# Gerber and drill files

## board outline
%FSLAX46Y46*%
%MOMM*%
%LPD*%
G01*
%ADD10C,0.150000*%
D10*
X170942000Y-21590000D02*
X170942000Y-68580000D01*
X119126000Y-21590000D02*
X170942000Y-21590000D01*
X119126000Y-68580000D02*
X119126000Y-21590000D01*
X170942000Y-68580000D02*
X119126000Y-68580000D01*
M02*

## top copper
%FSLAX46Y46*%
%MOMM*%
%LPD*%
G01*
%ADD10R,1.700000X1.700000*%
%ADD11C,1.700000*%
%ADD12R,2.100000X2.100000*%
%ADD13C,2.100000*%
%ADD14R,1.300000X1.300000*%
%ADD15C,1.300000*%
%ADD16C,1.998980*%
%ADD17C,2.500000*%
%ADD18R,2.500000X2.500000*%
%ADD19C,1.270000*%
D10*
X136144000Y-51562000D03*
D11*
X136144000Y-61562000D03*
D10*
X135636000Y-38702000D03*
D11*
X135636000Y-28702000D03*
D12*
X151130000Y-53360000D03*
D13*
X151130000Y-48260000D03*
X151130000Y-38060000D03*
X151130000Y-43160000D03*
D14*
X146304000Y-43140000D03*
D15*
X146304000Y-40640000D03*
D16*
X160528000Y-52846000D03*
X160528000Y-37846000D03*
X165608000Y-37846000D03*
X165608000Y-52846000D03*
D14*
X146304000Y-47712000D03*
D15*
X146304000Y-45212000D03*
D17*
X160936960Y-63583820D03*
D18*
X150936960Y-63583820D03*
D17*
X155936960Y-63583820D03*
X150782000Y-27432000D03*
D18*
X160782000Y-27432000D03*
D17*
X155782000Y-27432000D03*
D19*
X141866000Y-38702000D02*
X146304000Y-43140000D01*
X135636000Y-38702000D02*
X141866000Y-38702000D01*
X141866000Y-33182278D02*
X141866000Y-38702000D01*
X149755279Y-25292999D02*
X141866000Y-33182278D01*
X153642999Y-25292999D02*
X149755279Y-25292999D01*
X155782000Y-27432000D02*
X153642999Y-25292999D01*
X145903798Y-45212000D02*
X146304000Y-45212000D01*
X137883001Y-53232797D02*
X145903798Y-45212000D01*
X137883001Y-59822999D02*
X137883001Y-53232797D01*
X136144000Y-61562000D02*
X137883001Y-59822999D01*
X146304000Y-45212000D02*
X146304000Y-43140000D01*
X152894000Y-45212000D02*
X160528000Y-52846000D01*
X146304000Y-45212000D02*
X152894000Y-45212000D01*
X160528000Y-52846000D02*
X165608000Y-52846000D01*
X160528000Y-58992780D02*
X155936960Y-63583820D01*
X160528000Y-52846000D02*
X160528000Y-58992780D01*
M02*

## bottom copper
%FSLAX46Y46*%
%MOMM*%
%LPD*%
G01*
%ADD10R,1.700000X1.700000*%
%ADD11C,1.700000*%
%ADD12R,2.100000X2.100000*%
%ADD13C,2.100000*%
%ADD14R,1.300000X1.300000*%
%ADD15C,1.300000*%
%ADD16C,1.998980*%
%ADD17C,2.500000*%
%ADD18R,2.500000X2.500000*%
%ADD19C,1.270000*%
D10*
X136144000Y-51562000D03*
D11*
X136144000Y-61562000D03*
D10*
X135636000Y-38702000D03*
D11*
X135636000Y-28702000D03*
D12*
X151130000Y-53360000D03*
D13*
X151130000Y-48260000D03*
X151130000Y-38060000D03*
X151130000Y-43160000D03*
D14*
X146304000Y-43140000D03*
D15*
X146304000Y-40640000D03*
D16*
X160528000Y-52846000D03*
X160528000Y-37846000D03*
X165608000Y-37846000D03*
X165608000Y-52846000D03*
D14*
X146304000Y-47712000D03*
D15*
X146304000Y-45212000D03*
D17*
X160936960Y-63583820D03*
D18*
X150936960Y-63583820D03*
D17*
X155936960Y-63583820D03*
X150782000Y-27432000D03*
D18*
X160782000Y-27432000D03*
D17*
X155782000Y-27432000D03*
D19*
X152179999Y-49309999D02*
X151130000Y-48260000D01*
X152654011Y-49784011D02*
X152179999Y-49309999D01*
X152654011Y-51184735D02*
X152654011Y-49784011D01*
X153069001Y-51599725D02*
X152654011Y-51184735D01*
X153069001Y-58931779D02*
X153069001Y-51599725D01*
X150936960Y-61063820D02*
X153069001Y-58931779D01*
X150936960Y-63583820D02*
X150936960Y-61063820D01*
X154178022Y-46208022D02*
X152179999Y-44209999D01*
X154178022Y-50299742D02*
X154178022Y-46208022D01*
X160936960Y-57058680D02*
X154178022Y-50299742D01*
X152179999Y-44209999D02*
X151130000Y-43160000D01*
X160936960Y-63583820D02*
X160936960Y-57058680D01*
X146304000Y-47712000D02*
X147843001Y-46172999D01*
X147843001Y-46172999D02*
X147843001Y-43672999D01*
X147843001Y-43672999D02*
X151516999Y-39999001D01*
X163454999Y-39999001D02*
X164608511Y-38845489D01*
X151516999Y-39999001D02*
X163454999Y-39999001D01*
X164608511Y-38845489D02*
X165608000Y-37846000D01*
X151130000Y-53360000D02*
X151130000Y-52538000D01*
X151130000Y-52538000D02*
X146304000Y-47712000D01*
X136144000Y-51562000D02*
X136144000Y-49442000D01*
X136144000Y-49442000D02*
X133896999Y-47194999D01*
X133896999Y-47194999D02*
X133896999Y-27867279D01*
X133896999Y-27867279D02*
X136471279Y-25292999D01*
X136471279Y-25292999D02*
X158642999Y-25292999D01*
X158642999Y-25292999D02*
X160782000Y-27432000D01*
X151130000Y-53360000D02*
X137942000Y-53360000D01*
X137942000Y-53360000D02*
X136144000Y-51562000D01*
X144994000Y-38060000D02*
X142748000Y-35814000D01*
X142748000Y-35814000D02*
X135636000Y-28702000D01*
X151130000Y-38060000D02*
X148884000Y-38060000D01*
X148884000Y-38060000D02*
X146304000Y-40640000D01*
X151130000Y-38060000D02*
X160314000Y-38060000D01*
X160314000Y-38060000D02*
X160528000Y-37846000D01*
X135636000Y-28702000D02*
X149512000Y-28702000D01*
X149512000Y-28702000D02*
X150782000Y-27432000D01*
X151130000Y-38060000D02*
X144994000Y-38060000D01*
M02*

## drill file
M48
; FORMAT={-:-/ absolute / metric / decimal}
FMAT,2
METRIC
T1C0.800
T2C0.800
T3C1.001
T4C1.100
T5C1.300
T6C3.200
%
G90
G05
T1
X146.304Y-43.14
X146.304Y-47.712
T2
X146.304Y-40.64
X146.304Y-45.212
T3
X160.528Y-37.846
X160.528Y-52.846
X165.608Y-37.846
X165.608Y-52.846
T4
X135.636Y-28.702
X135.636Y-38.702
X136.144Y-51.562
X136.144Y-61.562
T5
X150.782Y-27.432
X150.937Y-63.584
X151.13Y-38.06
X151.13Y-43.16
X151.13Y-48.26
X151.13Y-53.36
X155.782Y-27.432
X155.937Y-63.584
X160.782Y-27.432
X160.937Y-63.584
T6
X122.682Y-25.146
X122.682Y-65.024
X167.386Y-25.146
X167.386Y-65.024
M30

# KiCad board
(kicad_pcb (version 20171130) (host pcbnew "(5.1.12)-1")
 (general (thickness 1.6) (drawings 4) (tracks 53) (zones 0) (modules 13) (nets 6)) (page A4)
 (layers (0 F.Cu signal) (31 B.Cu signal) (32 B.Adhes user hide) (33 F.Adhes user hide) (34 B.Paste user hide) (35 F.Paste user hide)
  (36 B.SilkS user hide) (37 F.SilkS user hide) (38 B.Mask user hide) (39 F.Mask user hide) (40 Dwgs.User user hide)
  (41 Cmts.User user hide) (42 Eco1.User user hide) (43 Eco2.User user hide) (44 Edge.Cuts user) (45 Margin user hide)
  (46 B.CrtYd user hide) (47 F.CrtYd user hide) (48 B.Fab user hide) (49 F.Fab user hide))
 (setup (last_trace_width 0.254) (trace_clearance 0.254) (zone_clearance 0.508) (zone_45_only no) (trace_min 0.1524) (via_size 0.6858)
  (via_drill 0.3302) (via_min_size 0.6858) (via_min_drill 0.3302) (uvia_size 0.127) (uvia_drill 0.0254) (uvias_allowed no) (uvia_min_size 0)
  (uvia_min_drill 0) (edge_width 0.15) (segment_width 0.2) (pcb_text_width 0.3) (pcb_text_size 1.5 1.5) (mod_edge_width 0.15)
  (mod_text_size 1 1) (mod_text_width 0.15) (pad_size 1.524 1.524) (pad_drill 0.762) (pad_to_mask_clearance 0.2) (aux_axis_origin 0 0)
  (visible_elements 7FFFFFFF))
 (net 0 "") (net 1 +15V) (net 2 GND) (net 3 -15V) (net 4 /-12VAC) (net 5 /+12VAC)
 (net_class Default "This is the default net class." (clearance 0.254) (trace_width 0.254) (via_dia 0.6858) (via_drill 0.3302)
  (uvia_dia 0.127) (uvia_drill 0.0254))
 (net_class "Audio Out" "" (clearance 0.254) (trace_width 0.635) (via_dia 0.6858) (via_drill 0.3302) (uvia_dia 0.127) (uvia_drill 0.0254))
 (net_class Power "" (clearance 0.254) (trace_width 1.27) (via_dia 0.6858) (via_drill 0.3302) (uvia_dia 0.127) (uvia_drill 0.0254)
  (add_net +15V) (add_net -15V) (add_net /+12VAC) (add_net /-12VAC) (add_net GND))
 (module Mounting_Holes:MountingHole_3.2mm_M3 (layer F.Cu) (at 122.682 25.146)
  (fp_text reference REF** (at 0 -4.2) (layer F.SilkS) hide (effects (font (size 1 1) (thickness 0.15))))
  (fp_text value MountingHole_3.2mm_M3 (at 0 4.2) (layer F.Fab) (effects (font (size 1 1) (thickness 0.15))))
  (pad 1 np_thru_hole circle (at 0 0) (size 3.2 3.2) (drill 3.2) (layers *.Cu *.Mask)))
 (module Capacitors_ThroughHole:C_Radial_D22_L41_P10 (layer F.Cu) (at 136.144 51.562 270)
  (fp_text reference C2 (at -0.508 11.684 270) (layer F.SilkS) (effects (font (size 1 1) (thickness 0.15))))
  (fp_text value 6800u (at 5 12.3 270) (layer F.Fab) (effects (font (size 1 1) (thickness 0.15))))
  (pad 1 thru_hole rect (at 0 0 270) (size 1.7 1.7) (drill 1.1) (layers *.Cu *.Mask) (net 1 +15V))
  (pad 2 thru_hole circle (at 10 0 270) (size 1.7 1.7) (drill 1.1) (layers *.Cu *.Mask) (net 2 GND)))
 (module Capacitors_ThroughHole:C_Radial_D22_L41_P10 (layer F.Cu) (at 135.636 38.702 90)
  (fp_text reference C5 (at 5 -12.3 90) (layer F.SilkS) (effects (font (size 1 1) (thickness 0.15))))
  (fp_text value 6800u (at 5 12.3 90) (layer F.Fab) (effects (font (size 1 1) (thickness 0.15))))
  (pad 1 thru_hole rect (at 0 0 90) (size 1.7 1.7) (drill 1.1) (layers *.Cu *.Mask) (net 2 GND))
  (pad 2 thru_hole circle (at 10 0 90) (size 1.7 1.7) (drill 1.1) (layers *.Cu *.Mask) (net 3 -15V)))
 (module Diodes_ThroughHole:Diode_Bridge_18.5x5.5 (layer F.Cu) (at 151.13 53.36 90)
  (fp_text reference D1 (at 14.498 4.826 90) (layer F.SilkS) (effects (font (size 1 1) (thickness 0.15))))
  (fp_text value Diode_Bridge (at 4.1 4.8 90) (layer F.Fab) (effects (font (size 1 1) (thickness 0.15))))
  (pad 3 thru_hole rect (at 0 0 90) (size 2.1 2.1) (drill 1.3) (layers *.Cu *.Mask) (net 1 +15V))
  (pad 2 thru_hole circle (at 5.1 0 90) (size 2.1 2.1) (drill 1.3) (layers *.Cu *.Mask) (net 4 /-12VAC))
  (pad 1 thru_hole circle (at 15.3 0 90) (size 2.1 2.1) (drill 1.3) (layers *.Cu *.Mask) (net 3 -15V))
  (pad 4 thru_hole circle (at 10.2 0 90) (size 2.1 2.1) (drill 1.3) (layers *.Cu *.Mask) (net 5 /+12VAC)))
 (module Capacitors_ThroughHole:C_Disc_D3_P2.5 (layer F.Cu) (at 146.304 43.14 90)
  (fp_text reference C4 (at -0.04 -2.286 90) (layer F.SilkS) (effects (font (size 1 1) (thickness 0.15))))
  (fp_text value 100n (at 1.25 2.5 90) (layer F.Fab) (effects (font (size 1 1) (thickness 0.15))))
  (pad 1 thru_hole rect (at 0 0 90) (size 1.3 1.3) (drill 0.8) (layers *.Cu *.Mask) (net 2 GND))
  (pad 2 thru_hole circle (at 2.5 0 90) (size 1.3 1.3) (drill 0.8001) (layers *.Cu *.Mask) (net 3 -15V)))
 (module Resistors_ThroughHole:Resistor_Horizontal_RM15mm (layer F.Cu) (at 160.528 52.846 90)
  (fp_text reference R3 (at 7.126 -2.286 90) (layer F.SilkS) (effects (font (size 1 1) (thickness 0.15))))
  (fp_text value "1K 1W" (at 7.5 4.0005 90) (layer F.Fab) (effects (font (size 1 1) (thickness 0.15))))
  (pad 1 thru_hole circle (at 0 0 90) (size 1.99898 1.99898) (drill 1.00076) (layers *.Cu *.SilkS *.Mask) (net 2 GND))
  (pad 2 thru_hole circle (at 15 0 90) (size 1.99898 1.99898) (drill 1.00076) (layers *.Cu *.SilkS *.Mask) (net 3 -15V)))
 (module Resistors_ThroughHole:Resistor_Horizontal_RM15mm (layer F.Cu) (at 165.608 37.846 270)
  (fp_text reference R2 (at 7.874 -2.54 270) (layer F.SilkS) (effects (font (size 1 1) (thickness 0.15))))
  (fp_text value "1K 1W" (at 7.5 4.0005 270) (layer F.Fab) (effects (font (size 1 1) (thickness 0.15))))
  (pad 1 thru_hole circle (at 0 0 270) (size 1.99898 1.99898) (drill 1.00076) (layers *.Cu *.SilkS *.Mask) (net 1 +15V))
  (pad 2 thru_hole circle (at 15 0 270) (size 1.99898 1.99898) (drill 1.00076) (layers *.Cu *.SilkS *.Mask) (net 2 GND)))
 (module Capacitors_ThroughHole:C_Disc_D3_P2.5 (layer F.Cu) (at 146.304 47.712 90)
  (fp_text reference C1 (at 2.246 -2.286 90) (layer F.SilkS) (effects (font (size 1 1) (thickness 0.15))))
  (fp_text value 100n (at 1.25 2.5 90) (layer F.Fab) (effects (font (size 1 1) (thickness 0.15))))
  (pad 1 thru_hole rect (at 0 0 90) (size 1.3 1.3) (drill 0.8) (layers *.Cu *.Mask) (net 1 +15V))
  (pad 2 thru_hole circle (at 2.5 0 90) (size 1.3 1.3) (drill 0.8001) (layers *.Cu *.Mask) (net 2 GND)))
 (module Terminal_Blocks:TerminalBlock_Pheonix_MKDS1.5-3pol (layer F.Cu) (at 150.93696 63.58382)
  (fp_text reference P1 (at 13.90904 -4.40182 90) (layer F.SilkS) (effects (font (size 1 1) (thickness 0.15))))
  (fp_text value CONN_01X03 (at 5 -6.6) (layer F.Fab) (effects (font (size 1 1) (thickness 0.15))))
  (pad 3 thru_hole circle (at 10 0) (size 2.5 2.5) (drill 1.3) (layers *.Cu *.Mask) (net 5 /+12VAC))
  (pad 1 thru_hole rect (at 0 0) (size 2.5 2.5) (drill 1.3) (layers *.Cu *.Mask) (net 4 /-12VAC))
  (pad 2 thru_hole circle (at 5 0) (size 2.5 2.5) (drill 1.3) (layers *.Cu *.Mask) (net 2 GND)))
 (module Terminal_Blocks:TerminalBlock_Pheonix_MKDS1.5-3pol (layer F.Cu) (at 160.782 27.432 180)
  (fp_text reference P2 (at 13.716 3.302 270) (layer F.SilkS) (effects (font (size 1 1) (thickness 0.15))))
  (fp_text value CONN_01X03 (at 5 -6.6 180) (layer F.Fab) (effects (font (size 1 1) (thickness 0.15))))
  (pad 3 thru_hole circle (at 10 0 180) (size 2.5 2.5) (drill 1.3) (layers *.Cu *.Mask) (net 3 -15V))
  (pad 1 thru_hole rect (at 0 0 180) (size 2.5 2.5) (drill 1.3) (layers *.Cu *.Mask) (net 1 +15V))
  (pad 2 thru_hole circle (at 5 0 180) (size 2.5 2.5) (drill 1.3) (layers *.Cu *.Mask) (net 2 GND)))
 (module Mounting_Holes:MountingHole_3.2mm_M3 (layer F.Cu) (at 167.386 25.146)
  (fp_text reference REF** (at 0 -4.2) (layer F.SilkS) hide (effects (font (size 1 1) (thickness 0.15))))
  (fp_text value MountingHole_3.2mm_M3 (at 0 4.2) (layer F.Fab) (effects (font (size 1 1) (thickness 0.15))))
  (pad 1 np_thru_hole circle (at 0 0) (size 3.2 3.2) (drill 3.2) (layers *.Cu *.Mask)))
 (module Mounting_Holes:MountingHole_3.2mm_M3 (layer F.Cu) (at 167.386 65.024)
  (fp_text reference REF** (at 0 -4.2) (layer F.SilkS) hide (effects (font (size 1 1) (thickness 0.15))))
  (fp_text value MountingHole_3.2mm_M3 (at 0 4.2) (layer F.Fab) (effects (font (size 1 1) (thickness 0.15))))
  (pad 1 np_thru_hole circle (at 0 0) (size 3.2 3.2) (drill 3.2) (layers *.Cu *.Mask)))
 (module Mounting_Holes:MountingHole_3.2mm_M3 (layer F.Cu) (at 122.682 65.024)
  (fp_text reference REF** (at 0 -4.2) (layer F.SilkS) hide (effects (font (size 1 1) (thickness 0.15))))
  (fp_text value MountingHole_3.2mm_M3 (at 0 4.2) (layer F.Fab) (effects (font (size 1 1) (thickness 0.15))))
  (pad 1 np_thru_hole circle (at 0 0) (size 3.2 3.2) (drill 3.2) (layers *.Cu *.Mask)))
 (gr_line (start 170.942 21.59) (end 170.942 68.58) (layer Edge.Cuts) (width 0.15))
 (gr_line (start 119.126 21.59) (end 170.942 21.59) (layer Edge.Cuts) (width 0.15))
 (gr_line (start 119.126 68.58) (end 119.126 21.59) (layer Edge.Cuts) (width 0.15))
 (gr_line (start 170.942 68.58) (end 119.126 68.58) (layer Edge.Cuts) (width 0.15))
 (segment (start 152.179999 49.309999) (end 151.13 48.26) (width 1.27) (layer B.Cu) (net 4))
 (segment (start 152.654011 49.784011) (end 152.179999 49.309999) (width 1.27) (layer B.Cu) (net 4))
 (segment (start 152.654011 51.184735) (end 152.654011 49.784011) (width 1.27) (layer B.Cu) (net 4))
 (segment (start 153.069001 51.599725) (end 152.654011 51.184735) (width 1.27) (layer B.Cu) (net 4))
 (segment (start 153.069001 58.931779) (end 153.069001 51.599725) (width 1.27) (layer B.Cu) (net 4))
 (segment (start 150.93696 61.06382) (end 153.069001 58.931779) (width 1.27) (layer B.Cu) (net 4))
 (segment (start 150.93696 63.58382) (end 150.93696 61.06382) (width 1.27) (layer B.Cu) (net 4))
 (segment (start 154.178022 46.208022) (end 152.179999 44.209999) (width 1.27) (layer B.Cu) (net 5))
 (segment (start 154.178022 50.299742) (end 154.178022 46.208022) (width 1.27) (layer B.Cu) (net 5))
 (segment (start 160.93696 57.05868) (end 154.178022 50.299742) (width 1.27) (layer B.Cu) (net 5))
 (segment (start 152.179999 44.209999) (end 151.13 43.16) (width 1.27) (layer B.Cu) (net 5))
 (segment (start 160.93696 63.58382) (end 160.93696 57.05868) (width 1.27) (layer B.Cu) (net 5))
 (segment (start 146.304 47.712) (end 147.843001 46.172999) (width 1.27) (layer B.Cu) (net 1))
 (segment (start 147.843001 46.172999) (end 147.843001 43.672999) (width 1.27) (layer B.Cu) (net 1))
 (segment (start 147.843001 43.672999) (end 151.516999 39.999001) (width 1.27) (layer B.Cu) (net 1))
 (segment (start 163.454999 39.999001) (end 164.608511 38.845489) (width 1.27) (layer B.Cu) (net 1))
 (segment (start 151.516999 39.999001) (end 163.454999 39.999001) (width 1.27) (layer B.Cu) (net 1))
 (segment (start 164.608511 38.845489) (end 165.608 37.846) (width 1.27) (layer B.Cu) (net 1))
 (segment (start 151.13 53.36) (end 151.13 52.538) (width 1.27) (layer B.Cu) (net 1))
 (segment (start 151.13 52.538) (end 146.304 47.712) (width 1.27) (layer B.Cu) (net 1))
 (segment (start 136.144 51.562) (end 136.144 49.442) (width 1.27) (layer B.Cu) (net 1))
 (segment (start 136.144 49.442) (end 133.896999 47.194999) (width 1.27) (layer B.Cu) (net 1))
 (segment (start 133.896999 47.194999) (end 133.896999 27.867279) (width 1.27) (layer B.Cu) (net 1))
 (segment (start 133.896999 27.867279) (end 136.471279 25.292999) (width 1.27) (layer B.Cu) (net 1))
 (segment (start 136.471279 25.292999) (end 158.642999 25.292999) (width 1.27) (layer B.Cu) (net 1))
 (segment (start 158.642999 25.292999) (end 160.782 27.432) (width 1.27) (layer B.Cu) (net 1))
 (segment (start 151.13 53.36) (end 137.942 53.36) (width 1.27) (layer B.Cu) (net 1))
 (segment (start 137.942 53.36) (end 136.144 51.562) (width 1.27) (layer B.Cu) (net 1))
 (segment (start 144.994 38.06) (end 142.748 35.814) (width 1.27) (layer B.Cu) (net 3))
 (segment (start 142.748 35.814) (end 135.636 28.702) (width 1.27) (layer B.Cu) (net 3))
 (segment (start 151.13 38.06) (end 148.884 38.06) (width 1.27) (layer B.Cu) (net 3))
 (segment (start 148.884 38.06) (end 146.304 40.64) (width 1.27) (layer B.Cu) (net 3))
 (segment (start 151.13 38.06) (end 160.314 38.06) (width 1.27) (layer B.Cu) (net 3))
 (segment (start 160.314 38.06) (end 160.528 37.846) (width 1.27) (layer B.Cu) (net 3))
 (segment (start 135.636 28.702) (end 149.512 28.702) (width 1.27) (layer B.Cu) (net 3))
 (segment (start 149.512 28.702) (end 150.782 27.432) (width 1.27) (layer B.Cu) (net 3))
 (segment (start 151.13 38.06) (end 144.994 38.06) (width 1.27) (layer B.Cu) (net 3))
 (segment (start 141.866 38.702) (end 146.304 43.14) (width 1.27) (layer F.Cu) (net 2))
 (segment (start 135.636 38.702) (end 141.866 38.702) (width 1.27) (layer F.Cu) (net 2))
 (segment (start 141.866 33.182278) (end 141.866 38.702) (width 1.27) (layer F.Cu) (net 2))
 (segment (start 149.755279 25.292999) (end 141.866 33.182278) (width 1.27) (layer F.Cu) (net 2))
 (segment (start 153.642999 25.292999) (end 149.755279 25.292999) (width 1.27) (layer F.Cu) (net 2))
 (segment (start 155.782 27.432) (end 153.642999 25.292999) (width 1.27) (layer F.Cu) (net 2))
 (segment (start 145.903798 45.212) (end 146.304 45.212) (width 1.27) (layer F.Cu) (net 2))
 (segment (start 137.883001 53.232797) (end 145.903798 45.212) (width 1.27) (layer F.Cu) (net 2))
 (segment (start 137.883001 59.822999) (end 137.883001 53.232797) (width 1.27) (layer F.Cu) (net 2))
 (segment (start 136.144 61.562) (end 137.883001 59.822999) (width 1.27) (layer F.Cu) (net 2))
 (segment (start 146.304 45.212) (end 146.304 43.14) (width 1.27) (layer F.Cu) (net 2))
 (segment (start 152.894 45.212) (end 160.528 52.846) (width 1.27) (layer F.Cu) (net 2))
 (segment (start 146.304 45.212) (end 152.894 45.212) (width 1.27) (layer F.Cu) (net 2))
 (segment (start 160.528 52.846) (end 165.608 52.846) (width 1.27) (layer F.Cu) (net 2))
 (segment (start 160.528 58.99278) (end 155.93696 63.58382) (width 1.27) (layer F.Cu) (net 2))
 (segment (start 160.528 52.846) (end 160.528 58.99278) (width 1.27) (layer F.Cu) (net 2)))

